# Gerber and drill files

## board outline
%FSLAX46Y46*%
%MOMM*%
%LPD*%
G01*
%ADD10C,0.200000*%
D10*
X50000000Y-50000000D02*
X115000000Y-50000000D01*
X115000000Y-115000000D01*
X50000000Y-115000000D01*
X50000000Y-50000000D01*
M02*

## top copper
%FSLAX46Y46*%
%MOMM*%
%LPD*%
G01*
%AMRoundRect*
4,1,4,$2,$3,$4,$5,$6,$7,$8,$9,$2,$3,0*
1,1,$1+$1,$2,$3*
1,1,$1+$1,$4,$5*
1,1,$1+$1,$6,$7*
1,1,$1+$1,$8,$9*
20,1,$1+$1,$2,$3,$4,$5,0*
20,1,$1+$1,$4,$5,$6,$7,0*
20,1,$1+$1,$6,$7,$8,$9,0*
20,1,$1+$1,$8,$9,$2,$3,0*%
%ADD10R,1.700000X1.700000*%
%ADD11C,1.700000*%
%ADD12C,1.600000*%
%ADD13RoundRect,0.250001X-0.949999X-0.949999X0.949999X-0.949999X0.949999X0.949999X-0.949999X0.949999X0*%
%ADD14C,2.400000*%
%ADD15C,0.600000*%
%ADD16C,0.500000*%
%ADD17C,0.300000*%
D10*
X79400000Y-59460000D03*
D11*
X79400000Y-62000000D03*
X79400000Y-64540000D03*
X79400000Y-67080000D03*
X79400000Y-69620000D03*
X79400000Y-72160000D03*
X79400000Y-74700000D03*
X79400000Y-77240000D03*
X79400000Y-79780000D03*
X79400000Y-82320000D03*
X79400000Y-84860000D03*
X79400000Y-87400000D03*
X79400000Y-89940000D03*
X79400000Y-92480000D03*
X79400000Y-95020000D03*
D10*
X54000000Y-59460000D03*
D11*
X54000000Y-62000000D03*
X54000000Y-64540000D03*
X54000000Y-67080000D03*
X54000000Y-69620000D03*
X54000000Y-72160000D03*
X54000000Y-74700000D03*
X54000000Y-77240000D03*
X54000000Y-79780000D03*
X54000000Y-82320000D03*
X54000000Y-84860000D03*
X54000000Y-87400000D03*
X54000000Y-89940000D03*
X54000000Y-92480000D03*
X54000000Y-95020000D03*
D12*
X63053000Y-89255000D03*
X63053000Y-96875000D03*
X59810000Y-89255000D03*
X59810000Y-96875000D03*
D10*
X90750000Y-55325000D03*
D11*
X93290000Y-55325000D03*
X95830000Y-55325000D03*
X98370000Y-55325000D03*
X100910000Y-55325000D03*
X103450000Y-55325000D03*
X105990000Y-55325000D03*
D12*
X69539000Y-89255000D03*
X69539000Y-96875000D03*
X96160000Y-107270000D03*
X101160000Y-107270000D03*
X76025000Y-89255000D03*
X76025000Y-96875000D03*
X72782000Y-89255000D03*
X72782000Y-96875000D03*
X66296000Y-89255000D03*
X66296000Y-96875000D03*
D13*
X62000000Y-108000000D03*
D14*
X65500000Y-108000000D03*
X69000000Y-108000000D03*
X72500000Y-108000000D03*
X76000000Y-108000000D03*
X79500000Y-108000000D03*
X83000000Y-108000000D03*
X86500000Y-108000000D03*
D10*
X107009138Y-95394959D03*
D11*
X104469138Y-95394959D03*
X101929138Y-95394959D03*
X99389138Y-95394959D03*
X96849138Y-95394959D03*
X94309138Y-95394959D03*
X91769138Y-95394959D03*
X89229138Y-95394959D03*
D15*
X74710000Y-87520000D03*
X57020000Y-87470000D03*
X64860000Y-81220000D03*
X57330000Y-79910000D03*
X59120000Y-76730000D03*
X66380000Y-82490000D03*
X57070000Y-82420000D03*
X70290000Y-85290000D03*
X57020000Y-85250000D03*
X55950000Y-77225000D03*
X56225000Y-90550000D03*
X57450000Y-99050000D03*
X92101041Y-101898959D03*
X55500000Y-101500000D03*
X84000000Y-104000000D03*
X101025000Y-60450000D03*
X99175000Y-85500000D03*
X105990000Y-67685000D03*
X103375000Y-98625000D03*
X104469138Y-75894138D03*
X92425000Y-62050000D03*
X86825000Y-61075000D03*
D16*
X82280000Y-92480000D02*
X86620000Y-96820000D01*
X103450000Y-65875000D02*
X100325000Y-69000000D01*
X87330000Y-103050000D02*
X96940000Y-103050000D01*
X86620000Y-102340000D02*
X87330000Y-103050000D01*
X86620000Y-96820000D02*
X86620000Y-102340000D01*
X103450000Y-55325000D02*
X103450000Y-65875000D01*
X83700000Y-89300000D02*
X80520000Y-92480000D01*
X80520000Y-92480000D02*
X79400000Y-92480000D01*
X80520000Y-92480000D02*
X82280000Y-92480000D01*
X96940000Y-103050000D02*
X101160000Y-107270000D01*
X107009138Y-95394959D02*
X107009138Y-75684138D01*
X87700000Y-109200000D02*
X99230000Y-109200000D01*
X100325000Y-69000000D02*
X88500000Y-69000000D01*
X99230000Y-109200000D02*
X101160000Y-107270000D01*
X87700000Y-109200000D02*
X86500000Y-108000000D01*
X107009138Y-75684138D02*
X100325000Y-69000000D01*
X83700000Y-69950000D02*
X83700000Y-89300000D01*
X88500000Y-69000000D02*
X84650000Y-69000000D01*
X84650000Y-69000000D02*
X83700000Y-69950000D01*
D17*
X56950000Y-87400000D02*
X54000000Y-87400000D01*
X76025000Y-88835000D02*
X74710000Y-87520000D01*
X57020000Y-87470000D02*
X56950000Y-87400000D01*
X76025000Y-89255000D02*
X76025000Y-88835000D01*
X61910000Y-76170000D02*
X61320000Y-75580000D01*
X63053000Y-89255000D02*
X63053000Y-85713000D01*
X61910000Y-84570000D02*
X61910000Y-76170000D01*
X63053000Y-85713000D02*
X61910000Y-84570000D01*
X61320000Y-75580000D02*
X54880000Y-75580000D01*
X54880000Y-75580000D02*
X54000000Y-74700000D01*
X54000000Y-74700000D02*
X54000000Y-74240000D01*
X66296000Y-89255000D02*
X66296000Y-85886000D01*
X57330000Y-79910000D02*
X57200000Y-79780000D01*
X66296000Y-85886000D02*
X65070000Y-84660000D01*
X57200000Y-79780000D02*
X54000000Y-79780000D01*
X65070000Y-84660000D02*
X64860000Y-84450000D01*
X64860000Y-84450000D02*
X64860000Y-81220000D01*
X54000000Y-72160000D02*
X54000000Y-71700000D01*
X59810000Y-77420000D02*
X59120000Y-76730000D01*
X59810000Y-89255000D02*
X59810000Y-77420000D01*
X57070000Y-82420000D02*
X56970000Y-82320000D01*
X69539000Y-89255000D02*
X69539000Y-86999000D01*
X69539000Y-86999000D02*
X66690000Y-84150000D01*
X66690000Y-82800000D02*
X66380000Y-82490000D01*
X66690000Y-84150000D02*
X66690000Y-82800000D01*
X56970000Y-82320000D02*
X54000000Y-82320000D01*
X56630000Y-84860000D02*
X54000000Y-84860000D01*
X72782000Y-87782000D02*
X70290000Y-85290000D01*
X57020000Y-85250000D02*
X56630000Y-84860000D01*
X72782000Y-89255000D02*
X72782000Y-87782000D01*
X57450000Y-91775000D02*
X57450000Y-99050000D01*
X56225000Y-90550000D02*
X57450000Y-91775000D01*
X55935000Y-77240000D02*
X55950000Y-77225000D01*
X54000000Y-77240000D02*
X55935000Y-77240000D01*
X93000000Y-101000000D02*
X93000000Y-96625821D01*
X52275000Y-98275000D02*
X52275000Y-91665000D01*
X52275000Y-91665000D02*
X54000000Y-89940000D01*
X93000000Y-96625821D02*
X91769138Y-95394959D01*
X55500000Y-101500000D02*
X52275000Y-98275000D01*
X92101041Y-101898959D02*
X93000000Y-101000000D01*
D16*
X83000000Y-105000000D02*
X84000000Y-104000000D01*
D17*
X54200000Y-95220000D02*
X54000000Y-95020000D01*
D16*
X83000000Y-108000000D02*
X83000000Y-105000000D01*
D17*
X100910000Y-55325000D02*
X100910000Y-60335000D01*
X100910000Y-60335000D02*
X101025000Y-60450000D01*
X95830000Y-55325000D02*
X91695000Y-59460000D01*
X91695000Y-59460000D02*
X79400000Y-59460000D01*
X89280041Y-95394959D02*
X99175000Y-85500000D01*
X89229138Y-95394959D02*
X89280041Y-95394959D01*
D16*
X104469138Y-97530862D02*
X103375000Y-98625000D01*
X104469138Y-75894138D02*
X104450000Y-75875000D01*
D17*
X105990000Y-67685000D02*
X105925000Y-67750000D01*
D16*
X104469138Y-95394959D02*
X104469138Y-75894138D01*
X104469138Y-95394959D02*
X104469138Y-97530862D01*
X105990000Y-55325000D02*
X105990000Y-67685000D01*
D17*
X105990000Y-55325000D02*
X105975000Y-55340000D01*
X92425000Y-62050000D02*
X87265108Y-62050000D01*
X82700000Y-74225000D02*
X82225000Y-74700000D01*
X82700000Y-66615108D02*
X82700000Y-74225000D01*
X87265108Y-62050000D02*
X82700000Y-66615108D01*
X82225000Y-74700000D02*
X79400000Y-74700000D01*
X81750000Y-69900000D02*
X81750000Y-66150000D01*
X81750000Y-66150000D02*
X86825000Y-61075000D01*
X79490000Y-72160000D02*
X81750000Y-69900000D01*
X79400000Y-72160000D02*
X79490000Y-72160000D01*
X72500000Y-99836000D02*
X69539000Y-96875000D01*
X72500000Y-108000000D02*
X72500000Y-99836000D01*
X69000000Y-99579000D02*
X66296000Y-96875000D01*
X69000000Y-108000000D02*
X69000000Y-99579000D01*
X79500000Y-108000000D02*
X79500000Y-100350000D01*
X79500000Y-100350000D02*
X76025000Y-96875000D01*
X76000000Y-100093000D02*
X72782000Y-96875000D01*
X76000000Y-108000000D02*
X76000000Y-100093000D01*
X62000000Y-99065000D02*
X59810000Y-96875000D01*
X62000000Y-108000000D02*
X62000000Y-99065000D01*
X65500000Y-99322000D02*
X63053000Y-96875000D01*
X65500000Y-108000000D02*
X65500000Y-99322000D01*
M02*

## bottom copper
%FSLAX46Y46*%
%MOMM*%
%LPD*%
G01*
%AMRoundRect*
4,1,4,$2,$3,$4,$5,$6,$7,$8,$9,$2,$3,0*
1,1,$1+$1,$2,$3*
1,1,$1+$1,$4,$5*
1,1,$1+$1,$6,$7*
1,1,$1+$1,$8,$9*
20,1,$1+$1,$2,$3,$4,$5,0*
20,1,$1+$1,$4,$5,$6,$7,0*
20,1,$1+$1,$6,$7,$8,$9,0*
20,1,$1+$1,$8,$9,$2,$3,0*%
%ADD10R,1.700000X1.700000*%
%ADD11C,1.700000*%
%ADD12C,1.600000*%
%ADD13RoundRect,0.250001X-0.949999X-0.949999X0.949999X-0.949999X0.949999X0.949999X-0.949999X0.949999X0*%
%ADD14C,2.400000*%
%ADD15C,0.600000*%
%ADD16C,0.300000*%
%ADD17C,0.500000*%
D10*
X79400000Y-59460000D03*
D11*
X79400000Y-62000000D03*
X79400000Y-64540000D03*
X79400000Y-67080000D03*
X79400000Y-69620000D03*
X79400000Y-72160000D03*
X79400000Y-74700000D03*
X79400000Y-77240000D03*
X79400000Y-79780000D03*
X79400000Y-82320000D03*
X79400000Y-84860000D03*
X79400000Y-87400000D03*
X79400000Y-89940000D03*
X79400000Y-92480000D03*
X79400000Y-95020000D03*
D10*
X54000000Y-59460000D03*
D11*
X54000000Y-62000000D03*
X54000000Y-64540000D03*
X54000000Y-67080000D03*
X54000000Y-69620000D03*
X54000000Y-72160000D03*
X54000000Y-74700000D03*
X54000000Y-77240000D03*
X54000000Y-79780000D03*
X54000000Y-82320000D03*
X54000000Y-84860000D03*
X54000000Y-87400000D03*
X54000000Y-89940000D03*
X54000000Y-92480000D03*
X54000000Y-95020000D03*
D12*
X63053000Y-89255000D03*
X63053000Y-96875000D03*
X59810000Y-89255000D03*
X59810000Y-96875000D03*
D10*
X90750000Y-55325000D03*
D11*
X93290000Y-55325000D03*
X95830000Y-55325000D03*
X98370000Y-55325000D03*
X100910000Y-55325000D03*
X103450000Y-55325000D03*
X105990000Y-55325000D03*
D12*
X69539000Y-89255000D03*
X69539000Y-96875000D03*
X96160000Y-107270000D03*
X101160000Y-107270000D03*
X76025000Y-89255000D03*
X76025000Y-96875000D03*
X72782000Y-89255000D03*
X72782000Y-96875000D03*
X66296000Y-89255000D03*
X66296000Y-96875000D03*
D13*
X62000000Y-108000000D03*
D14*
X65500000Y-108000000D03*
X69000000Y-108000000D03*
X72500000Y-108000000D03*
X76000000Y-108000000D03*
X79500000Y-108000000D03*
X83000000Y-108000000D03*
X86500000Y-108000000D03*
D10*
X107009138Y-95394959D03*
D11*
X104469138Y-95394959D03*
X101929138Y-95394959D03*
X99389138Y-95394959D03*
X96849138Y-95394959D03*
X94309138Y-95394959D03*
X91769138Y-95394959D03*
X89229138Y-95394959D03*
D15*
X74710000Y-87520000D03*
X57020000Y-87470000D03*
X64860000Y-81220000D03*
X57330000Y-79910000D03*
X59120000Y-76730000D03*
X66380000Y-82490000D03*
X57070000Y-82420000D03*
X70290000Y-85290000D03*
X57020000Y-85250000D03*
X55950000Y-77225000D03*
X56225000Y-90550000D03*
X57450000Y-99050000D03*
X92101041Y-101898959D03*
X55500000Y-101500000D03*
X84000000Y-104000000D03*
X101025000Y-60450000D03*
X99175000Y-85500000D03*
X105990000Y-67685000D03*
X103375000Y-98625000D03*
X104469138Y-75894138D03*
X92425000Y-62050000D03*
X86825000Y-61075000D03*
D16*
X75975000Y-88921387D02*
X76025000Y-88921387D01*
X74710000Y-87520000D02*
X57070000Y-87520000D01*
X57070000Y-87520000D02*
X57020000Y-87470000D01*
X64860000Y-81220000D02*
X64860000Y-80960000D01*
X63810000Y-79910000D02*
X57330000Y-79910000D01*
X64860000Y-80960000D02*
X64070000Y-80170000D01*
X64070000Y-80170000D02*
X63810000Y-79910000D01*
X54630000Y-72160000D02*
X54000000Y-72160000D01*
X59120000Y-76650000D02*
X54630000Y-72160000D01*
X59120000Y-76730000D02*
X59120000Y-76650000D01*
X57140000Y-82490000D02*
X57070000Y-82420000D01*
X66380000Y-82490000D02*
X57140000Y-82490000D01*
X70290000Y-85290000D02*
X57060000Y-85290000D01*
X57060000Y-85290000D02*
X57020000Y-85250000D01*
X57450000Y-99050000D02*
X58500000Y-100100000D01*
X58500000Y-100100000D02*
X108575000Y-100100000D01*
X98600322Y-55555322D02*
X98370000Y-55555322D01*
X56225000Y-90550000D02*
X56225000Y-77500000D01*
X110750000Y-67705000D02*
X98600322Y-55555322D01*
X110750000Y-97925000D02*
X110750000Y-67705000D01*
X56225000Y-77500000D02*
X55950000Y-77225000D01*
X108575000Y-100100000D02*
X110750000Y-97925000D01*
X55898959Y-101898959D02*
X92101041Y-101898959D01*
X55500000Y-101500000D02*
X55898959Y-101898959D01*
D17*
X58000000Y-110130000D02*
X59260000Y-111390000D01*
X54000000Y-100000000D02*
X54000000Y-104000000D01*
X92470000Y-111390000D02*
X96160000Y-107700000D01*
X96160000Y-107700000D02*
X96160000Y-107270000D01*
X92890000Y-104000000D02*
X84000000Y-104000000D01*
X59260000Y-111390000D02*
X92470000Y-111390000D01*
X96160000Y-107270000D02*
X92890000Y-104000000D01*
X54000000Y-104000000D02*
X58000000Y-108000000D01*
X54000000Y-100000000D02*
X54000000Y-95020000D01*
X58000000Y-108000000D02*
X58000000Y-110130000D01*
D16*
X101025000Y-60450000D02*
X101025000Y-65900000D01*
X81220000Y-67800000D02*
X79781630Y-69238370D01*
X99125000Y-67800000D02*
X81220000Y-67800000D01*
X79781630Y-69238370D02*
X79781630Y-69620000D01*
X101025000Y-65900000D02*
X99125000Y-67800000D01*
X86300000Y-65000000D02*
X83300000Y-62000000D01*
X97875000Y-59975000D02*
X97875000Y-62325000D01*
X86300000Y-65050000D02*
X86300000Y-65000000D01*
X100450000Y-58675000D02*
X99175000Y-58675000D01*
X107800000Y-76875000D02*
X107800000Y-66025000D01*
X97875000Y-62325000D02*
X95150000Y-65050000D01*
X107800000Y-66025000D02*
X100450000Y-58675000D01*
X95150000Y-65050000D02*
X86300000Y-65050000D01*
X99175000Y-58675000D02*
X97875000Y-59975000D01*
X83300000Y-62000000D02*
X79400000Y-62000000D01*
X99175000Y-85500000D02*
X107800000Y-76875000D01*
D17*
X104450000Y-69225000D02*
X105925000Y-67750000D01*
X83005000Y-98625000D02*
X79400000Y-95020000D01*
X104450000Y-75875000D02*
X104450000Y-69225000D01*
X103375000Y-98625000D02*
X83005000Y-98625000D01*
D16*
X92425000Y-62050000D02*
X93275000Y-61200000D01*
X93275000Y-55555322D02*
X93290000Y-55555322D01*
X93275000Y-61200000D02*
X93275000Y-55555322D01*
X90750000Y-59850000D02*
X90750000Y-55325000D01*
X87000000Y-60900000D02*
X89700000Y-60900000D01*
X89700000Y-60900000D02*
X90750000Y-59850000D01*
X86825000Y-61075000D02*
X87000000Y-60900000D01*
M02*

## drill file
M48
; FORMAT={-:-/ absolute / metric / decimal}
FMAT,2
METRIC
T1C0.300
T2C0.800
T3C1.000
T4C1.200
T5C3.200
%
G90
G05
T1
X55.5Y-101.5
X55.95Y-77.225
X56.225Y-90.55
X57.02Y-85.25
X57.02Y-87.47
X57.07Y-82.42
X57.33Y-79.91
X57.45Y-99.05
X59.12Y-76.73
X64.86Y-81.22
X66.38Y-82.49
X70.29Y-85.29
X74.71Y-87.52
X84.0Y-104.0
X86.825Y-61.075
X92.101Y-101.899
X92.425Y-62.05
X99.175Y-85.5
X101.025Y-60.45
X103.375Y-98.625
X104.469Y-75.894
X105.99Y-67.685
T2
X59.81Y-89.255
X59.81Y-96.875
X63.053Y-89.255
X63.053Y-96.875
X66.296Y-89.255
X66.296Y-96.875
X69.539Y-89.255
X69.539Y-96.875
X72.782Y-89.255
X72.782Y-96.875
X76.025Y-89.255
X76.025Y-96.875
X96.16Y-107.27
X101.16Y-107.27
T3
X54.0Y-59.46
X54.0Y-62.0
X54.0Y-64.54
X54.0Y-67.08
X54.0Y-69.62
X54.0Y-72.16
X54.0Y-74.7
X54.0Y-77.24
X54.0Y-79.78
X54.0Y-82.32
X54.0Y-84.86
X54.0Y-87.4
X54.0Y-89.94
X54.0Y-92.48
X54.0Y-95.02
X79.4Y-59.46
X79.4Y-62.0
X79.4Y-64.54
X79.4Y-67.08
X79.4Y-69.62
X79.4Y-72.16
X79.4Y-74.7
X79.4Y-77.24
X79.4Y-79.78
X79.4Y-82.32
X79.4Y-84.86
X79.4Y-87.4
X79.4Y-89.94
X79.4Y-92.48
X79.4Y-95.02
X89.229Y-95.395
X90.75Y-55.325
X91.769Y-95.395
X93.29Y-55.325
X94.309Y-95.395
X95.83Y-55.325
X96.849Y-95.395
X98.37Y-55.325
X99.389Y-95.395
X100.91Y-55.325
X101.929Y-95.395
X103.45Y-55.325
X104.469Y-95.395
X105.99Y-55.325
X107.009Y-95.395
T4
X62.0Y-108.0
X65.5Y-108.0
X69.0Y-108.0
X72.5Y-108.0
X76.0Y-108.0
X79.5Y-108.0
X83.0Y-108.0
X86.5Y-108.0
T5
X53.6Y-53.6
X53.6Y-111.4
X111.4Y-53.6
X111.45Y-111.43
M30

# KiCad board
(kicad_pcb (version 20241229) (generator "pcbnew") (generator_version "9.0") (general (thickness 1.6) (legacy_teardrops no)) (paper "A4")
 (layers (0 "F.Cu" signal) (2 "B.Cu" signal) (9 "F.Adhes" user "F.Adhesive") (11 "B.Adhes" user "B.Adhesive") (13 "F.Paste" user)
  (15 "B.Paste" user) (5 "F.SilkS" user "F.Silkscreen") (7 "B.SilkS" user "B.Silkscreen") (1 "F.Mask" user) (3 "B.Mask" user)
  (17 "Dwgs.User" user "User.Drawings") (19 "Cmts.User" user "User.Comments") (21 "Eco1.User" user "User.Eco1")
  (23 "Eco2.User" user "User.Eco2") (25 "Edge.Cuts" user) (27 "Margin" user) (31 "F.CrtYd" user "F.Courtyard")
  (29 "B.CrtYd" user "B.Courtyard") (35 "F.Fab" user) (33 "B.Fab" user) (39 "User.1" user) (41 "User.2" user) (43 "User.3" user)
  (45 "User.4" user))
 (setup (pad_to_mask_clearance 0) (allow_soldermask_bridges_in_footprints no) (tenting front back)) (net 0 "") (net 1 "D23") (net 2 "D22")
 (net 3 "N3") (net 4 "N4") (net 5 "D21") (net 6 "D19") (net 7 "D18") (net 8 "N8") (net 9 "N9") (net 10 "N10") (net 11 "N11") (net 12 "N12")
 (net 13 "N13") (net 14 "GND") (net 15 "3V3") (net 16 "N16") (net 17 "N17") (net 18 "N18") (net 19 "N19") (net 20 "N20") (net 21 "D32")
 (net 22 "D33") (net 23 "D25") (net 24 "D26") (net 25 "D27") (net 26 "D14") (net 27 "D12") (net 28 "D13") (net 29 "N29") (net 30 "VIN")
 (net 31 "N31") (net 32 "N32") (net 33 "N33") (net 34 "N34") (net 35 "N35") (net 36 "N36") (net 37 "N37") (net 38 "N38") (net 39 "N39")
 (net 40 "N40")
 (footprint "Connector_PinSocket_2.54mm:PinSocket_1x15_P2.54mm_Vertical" (layer "F.Cu") (at 79.4 59.46)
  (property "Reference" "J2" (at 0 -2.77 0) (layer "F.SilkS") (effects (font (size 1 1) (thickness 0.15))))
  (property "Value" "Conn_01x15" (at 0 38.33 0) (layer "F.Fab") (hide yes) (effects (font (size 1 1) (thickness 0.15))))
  (pad "1" thru_hole rect (at 0 0) (size 1.7 1.7) (drill 1) (layers "*.Cu" "*.Mask") (remove_unused_layers no) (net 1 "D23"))
  (pad "2" thru_hole circle (at 0 2.54) (size 1.7 1.7) (drill 1) (layers "*.Cu" "*.Mask") (remove_unused_layers no) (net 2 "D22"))
  (pad "3" thru_hole circle (at 0 5.08) (size 1.7 1.7) (drill 1) (layers "*.Cu" "*.Mask") (remove_unused_layers no) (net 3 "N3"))
  (pad "4" thru_hole circle (at 0 7.62) (size 1.7 1.7) (drill 1) (layers "*.Cu" "*.Mask") (remove_unused_layers no) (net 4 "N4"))
  (pad "5" thru_hole circle (at 0 10.16) (size 1.7 1.7) (drill 1) (layers "*.Cu" "*.Mask") (remove_unused_layers no) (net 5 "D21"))
  (pad "6" thru_hole circle (at 0 12.7) (size 1.7 1.7) (drill 1) (layers "*.Cu" "*.Mask") (remove_unused_layers no) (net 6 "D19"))
  (pad "7" thru_hole circle (at 0 15.24) (size 1.7 1.7) (drill 1) (layers "*.Cu" "*.Mask") (remove_unused_layers no) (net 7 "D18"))
  (pad "8" thru_hole circle (at 0 17.78) (size 1.7 1.7) (drill 1) (layers "*.Cu" "*.Mask") (remove_unused_layers no) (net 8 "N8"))
  (pad "9" thru_hole circle (at 0 20.32) (size 1.7 1.7) (drill 1) (layers "*.Cu" "*.Mask") (remove_unused_layers no) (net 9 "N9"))
  (pad "10" thru_hole circle (at 0 22.86) (size 1.7 1.7) (drill 1) (layers "*.Cu" "*.Mask") (remove_unused_layers no) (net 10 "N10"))
  (pad "11" thru_hole circle (at 0 25.4) (size 1.7 1.7) (drill 1) (layers "*.Cu" "*.Mask") (remove_unused_layers no) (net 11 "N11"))
  (pad "12" thru_hole circle (at 0 27.94) (size 1.7 1.7) (drill 1) (layers "*.Cu" "*.Mask") (remove_unused_layers no) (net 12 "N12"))
  (pad "13" thru_hole circle (at 0 30.48) (size 1.7 1.7) (drill 1) (layers "*.Cu" "*.Mask") (remove_unused_layers no) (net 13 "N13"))
  (pad "14" thru_hole circle (at 0 33.02) (size 1.7 1.7) (drill 1) (layers "*.Cu" "*.Mask") (remove_unused_layers no) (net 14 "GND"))
  (pad "15" thru_hole circle (at 0 35.56) (size 1.7 1.7) (drill 1) (layers "*.Cu" "*.Mask") (remove_unused_layers no) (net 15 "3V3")))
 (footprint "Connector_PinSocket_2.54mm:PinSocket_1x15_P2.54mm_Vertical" (layer "F.Cu") (at 54 59.46)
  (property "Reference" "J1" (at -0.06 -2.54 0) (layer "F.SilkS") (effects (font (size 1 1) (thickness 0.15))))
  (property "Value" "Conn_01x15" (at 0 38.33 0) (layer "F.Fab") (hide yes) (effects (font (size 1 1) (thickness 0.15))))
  (pad "1" thru_hole rect (at 0 0) (size 1.7 1.7) (drill 1) (layers "*.Cu" "*.Mask") (remove_unused_layers no) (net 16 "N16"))
  (pad "2" thru_hole circle (at 0 2.54) (size 1.7 1.7) (drill 1) (layers "*.Cu" "*.Mask") (remove_unused_layers no) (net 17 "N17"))
  (pad "3" thru_hole circle (at 0 5.08) (size 1.7 1.7) (drill 1) (layers "*.Cu" "*.Mask") (remove_unused_layers no) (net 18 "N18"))
  (pad "4" thru_hole circle (at 0 7.62) (size 1.7 1.7) (drill 1) (layers "*.Cu" "*.Mask") (remove_unused_layers no) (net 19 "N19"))
  (pad "5" thru_hole circle (at 0 10.16) (size 1.7 1.7) (drill 1) (layers "*.Cu" "*.Mask") (remove_unused_layers no) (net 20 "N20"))
  (pad "6" thru_hole circle (at 0 12.7) (size 1.7 1.7) (drill 1) (layers "*.Cu" "*.Mask") (remove_unused_layers no) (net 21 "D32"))
  (pad "7" thru_hole circle (at 0 15.24) (size 1.7 1.7) (drill 1) (layers "*.Cu" "*.Mask") (remove_unused_layers no) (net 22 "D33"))
  (pad "8" thru_hole circle (at 0 17.78) (size 1.7 1.7) (drill 1) (layers "*.Cu" "*.Mask") (remove_unused_layers no) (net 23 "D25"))
  (pad "9" thru_hole circle (at 0 20.32) (size 1.7 1.7) (drill 1) (layers "*.Cu" "*.Mask") (remove_unused_layers no) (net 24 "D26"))
  (pad "10" thru_hole circle (at 0 22.86) (size 1.7 1.7) (drill 1) (layers "*.Cu" "*.Mask") (remove_unused_layers no) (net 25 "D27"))
  (pad "11" thru_hole circle (at 0 25.4) (size 1.7 1.7) (drill 1) (layers "*.Cu" "*.Mask") (remove_unused_layers no) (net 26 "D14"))
  (pad "12" thru_hole circle (at 0 27.94) (size 1.7 1.7) (drill 1) (layers "*.Cu" "*.Mask") (remove_unused_layers no) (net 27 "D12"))
  (pad "13" thru_hole circle (at 0 30.48) (size 1.7 1.7) (drill 1) (layers "*.Cu" "*.Mask") (remove_unused_layers no) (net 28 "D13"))
  (pad "14" thru_hole circle (at 0 33.02) (size 1.7 1.7) (drill 1) (layers "*.Cu" "*.Mask") (remove_unused_layers no) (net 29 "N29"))
  (pad "15" thru_hole circle (at 0 35.56) (size 1.7 1.7) (drill 1) (layers "*.Cu" "*.Mask") (remove_unused_layers no) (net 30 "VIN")))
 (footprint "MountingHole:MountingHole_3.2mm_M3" (layer "F.Cu") (at 53.6 53.6)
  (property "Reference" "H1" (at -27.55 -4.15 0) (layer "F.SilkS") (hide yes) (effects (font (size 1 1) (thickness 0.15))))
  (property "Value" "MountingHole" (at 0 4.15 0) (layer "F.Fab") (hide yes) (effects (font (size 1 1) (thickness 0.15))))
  (pad "" np_thru_hole circle (at 0 0) (size 3.2 3.2) (drill 3.2) (layers "*.Cu" "*.Mask")))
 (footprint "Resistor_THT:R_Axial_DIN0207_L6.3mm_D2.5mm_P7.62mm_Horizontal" (layer "F.Cu") (at 63.053 89.255 -90)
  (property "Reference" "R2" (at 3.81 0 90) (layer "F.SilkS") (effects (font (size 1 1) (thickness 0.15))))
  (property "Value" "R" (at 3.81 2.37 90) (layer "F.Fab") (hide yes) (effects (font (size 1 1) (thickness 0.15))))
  (pad "1" thru_hole circle (at 0 0 270) (size 1.6 1.6) (drill 0.8) (layers "*.Cu" "*.Mask") (remove_unused_layers no) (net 22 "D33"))
  (pad "2" thru_hole circle (at 7.62 0 270) (size 1.6 1.6) (drill 0.8) (layers "*.Cu" "*.Mask") (remove_unused_layers no) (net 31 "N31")))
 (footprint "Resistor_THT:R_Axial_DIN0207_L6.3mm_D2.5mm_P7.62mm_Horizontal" (layer "F.Cu") (at 59.81 89.255 -90)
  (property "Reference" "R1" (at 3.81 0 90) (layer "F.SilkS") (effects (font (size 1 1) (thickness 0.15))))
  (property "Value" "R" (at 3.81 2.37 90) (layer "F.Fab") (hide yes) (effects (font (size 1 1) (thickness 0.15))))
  (pad "1" thru_hole circle (at 0 0 270) (size 1.6 1.6) (drill 0.8) (layers "*.Cu" "*.Mask") (remove_unused_layers no) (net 21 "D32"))
  (pad "2" thru_hole circle (at 7.62 0 270) (size 1.6 1.6) (drill 0.8) (layers "*.Cu" "*.Mask") (remove_unused_layers no) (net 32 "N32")))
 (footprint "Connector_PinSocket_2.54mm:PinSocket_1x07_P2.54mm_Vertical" (layer "F.Cu") (at 90.75 55.325 90)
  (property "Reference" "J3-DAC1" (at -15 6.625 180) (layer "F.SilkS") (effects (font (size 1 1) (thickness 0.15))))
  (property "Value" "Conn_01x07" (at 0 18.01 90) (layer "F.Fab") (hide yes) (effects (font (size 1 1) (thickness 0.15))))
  (pad "1" thru_hole rect (at 0 0 90) (size 1.7 1.7) (drill 1) (layers "*.Cu" "*.Mask") (remove_unused_layers no) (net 6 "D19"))
  (pad "2" thru_hole circle (at 0 2.54 90) (size 1.7 1.7) (drill 1) (layers "*.Cu" "*.Mask") (remove_unused_layers no) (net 7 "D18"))
  (pad "3" thru_hole circle (at 0 5.08 90) (size 1.7 1.7) (drill 1) (layers "*.Cu" "*.Mask") (remove_unused_layers no) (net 1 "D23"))
  (pad "4" thru_hole circle (at 0 7.62 90) (size 1.7 1.7) (drill 1) (layers "*.Cu" "*.Mask") (remove_unused_layers no) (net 23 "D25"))
  (pad "5" thru_hole circle (at 0 10.16 90) (size 1.7 1.7) (drill 1) (layers "*.Cu" "*.Mask") (remove_unused_layers no) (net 5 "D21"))
  (pad "6" thru_hole circle (at 0 12.7 90) (size 1.7 1.7) (drill 1) (layers "*.Cu" "*.Mask") (remove_unused_layers no) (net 14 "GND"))
  (pad "7" thru_hole circle (at 0 15.24 90) (size 1.7 1.7) (drill 1) (layers "*.Cu" "*.Mask") (remove_unused_layers no) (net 15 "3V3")))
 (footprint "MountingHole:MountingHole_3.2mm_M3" (layer "F.Cu") (at 53.6 111.4)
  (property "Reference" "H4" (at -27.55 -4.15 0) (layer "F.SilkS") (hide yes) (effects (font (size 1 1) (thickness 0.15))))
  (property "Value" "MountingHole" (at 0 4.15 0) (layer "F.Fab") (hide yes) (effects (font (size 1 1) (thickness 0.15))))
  (pad "" np_thru_hole circle (at 0 0) (size 3.2 3.2) (drill 3.2) (layers "*.Cu" "*.Mask")))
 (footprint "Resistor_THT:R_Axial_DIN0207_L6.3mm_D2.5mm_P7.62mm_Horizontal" (layer "F.Cu") (at 69.539 89.255 -90)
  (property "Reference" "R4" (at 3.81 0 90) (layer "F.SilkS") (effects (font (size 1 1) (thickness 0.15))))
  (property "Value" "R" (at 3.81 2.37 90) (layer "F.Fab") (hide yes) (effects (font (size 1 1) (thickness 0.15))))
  (pad "1" thru_hole circle (at 0 0 270) (size 1.6 1.6) (drill 0.8) (layers "*.Cu" "*.Mask") (remove_unused_layers no) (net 25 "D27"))
  (pad "2" thru_hole circle (at 7.62 0 270) (size 1.6 1.6) (drill 0.8) (layers "*.Cu" "*.Mask") (remove_unused_layers no) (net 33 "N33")))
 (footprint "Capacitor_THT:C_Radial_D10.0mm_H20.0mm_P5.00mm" (layer "F.Cu") (at 96.16 107.27)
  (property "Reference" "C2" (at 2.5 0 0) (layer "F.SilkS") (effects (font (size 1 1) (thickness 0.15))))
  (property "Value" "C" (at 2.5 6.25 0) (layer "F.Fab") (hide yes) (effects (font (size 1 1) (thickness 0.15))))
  (pad "1" thru_hole circle (at 0 0) (size 1.6 1.6) (drill 0.8) (layers "*.Cu" "*.Mask") (remove_unused_layers no) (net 30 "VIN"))
  (pad "2" thru_hole circle (at 5 0) (size 1.6 1.6) (drill 0.8) (layers "*.Cu" "*.Mask") (remove_unused_layers no) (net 14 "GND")))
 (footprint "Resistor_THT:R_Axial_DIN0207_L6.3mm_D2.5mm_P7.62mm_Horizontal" (layer "F.Cu") (at 76.025 89.255 -90)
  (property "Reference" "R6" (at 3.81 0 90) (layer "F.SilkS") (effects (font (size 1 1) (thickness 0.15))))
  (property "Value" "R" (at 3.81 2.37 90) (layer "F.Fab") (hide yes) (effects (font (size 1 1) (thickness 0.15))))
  (pad "1" thru_hole circle (at 0 0 270) (size 1.6 1.6) (drill 0.8) (layers "*.Cu" "*.Mask") (remove_unused_layers no) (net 27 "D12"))
  (pad "2" thru_hole circle (at 7.62 0 270) (size 1.6 1.6) (drill 0.8) (layers "*.Cu" "*.Mask") (remove_unused_layers no) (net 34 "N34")))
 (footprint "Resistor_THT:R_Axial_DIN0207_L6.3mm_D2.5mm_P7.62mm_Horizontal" (layer "F.Cu") (at 72.782 89.255 -90)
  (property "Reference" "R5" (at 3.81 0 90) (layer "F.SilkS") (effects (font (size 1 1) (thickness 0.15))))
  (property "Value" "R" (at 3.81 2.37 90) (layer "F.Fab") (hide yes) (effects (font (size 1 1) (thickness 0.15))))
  (pad "1" thru_hole circle (at 0 0 270) (size 1.6 1.6) (drill 0.8) (layers "*.Cu" "*.Mask") (remove_unused_layers no) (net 26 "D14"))
  (pad "2" thru_hole circle (at 7.62 0 270) (size 1.6 1.6) (drill 0.8) (layers "*.Cu" "*.Mask") (remove_unused_layers no) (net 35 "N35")))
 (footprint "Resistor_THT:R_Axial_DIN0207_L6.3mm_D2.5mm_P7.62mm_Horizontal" (layer "F.Cu") (at 66.296 89.255 -90)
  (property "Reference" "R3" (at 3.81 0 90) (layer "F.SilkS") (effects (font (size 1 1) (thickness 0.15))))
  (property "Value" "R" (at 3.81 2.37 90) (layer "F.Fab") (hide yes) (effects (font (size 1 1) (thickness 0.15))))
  (pad "1" thru_hole circle (at 0 0 270) (size 1.6 1.6) (drill 0.8) (layers "*.Cu" "*.Mask") (remove_unused_layers no) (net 24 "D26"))
  (pad "2" thru_hole circle (at 7.62 0 270) (size 1.6 1.6) (drill 0.8) (layers "*.Cu" "*.Mask") (remove_unused_layers no) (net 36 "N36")))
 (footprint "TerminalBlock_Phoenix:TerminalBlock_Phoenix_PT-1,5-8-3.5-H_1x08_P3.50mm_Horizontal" (layer "F.Cu") (at 62 108)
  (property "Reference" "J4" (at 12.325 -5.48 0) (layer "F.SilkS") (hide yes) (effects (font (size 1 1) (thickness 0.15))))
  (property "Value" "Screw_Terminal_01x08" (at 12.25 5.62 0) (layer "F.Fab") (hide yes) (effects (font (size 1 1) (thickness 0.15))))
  (pad "1" thru_hole roundrect (at 0 0) (size 2.4 2.4) (drill 1.2) (layers "*.Cu" "*.Mask") (remove_unused_layers no)
   (roundrect_rratio 0.104167) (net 32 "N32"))
  (pad "2" thru_hole circle (at 3.5 0) (size 2.4 2.4) (drill 1.2) (layers "*.Cu" "*.Mask") (remove_unused_layers no) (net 31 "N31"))
  (pad "3" thru_hole circle (at 7 0) (size 2.4 2.4) (drill 1.2) (layers "*.Cu" "*.Mask") (remove_unused_layers no) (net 36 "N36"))
  (pad "4" thru_hole circle (at 10.5 0) (size 2.4 2.4) (drill 1.2) (layers "*.Cu" "*.Mask") (remove_unused_layers no) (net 33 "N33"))
  (pad "5" thru_hole circle (at 14 0) (size 2.4 2.4) (drill 1.2) (layers "*.Cu" "*.Mask") (remove_unused_layers no) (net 35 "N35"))
  (pad "6" thru_hole circle (at 17.5 0) (size 2.4 2.4) (drill 1.2) (layers "*.Cu" "*.Mask") (remove_unused_layers no) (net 34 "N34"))
  (pad "7" thru_hole circle (at 21 0) (size 2.4 2.4) (drill 1.2) (layers "*.Cu" "*.Mask") (remove_unused_layers no) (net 30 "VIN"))
  (pad "8" thru_hole circle (at 24.5 0) (size 2.4 2.4) (drill 1.2) (layers "*.Cu" "*.Mask") (remove_unused_layers no) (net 14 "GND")))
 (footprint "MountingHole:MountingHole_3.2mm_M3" (layer "F.Cu") (at 111.45 111.43)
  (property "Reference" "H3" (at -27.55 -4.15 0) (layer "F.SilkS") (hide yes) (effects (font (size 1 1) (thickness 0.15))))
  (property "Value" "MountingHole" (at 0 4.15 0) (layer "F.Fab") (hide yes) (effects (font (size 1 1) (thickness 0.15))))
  (pad "" np_thru_hole circle (at 0 0) (size 3.2 3.2) (drill 3.2) (layers "*.Cu" "*.Mask")))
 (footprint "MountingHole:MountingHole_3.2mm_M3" (layer "F.Cu") (at 111.4 53.6)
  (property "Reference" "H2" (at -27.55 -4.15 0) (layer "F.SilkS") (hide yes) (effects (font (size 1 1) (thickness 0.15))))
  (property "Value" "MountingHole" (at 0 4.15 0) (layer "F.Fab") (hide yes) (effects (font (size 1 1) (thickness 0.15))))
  (pad "" np_thru_hole circle (at 0 0) (size 3.2 3.2) (drill 3.2) (layers "*.Cu" "*.Mask")))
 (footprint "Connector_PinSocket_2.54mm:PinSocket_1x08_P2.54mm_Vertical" (layer "F.Cu") (at 107.009138 95.394959 -90)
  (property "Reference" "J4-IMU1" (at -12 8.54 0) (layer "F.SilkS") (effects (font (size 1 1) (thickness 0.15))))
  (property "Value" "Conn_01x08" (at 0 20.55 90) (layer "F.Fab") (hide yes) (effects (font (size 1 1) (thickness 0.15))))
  (pad "1" thru_hole rect (at 0 0 270) (size 1.7 1.7) (drill 1) (layers "*.Cu" "*.Mask") (remove_unused_layers no) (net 14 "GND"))
  (pad "2" thru_hole circle (at 0 2.54 270) (size 1.7 1.7) (drill 1) (layers "*.Cu" "*.Mask") (remove_unused_layers no) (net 15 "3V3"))
  (pad "3" thru_hole circle (at 0 5.08 270) (size 1.7 1.7) (drill 1) (layers "*.Cu" "*.Mask") (remove_unused_layers no) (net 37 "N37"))
  (pad "4" thru_hole circle (at 0 7.62 270) (size 1.7 1.7) (drill 1) (layers "*.Cu" "*.Mask") (remove_unused_layers no) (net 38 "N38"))
  (pad "5" thru_hole circle (at 0 10.16 270) (size 1.7 1.7) (drill 1) (layers "*.Cu" "*.Mask") (remove_unused_layers no) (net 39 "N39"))
  (pad "6" thru_hole circle (at 0 12.7 270) (size 1.7 1.7) (drill 1) (layers "*.Cu" "*.Mask") (remove_unused_layers no) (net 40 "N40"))
  (pad "7" thru_hole circle (at 0 15.24 270) (size 1.7 1.7) (drill 1) (layers "*.Cu" "*.Mask") (remove_unused_layers no) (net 28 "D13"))
  (pad "8" thru_hole circle (at 0 17.78 270) (size 1.7 1.7) (drill 1) (layers "*.Cu" "*.Mask") (remove_unused_layers no) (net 2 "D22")))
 (gr_rect (start 50 50) (end 115 115) (stroke (width 0.2) (type solid)) (fill no) (layer "Edge.Cuts"))
 (segment (start 82.28 92.48) (end 86.62 96.82) (width 0.5) (layer "F.Cu") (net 14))
 (segment (start 103.45 65.875) (end 100.325 69) (width 0.5) (layer "F.Cu") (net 14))
 (segment (start 87.33 103.05) (end 96.94 103.05) (width 0.5) (layer "F.Cu") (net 14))
 (segment (start 86.62 102.34) (end 87.33 103.05) (width 0.5) (layer "F.Cu") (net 14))
 (segment (start 86.62 96.82) (end 86.62 102.34) (width 0.5) (layer "F.Cu") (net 14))
 (segment (start 103.45 55.325) (end 103.45 65.875) (width 0.5) (layer "F.Cu") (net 14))
 (segment (start 83.7 89.3) (end 80.52 92.48) (width 0.5) (layer "F.Cu") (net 14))
 (segment (start 80.52 92.48) (end 79.4 92.48) (width 0.5) (layer "F.Cu") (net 14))
 (segment (start 80.52 92.48) (end 82.28 92.48) (width 0.5) (layer "F.Cu") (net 14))
 (segment (start 96.94 103.05) (end 101.16 107.27) (width 0.5) (layer "F.Cu") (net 14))
 (segment (start 107.009138 95.394959) (end 107.009138 75.684138) (width 0.5) (layer "F.Cu") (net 14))
 (segment (start 87.7 109.2) (end 99.23 109.2) (width 0.5) (layer "F.Cu") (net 14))
 (segment (start 100.325 69) (end 88.5 69) (width 0.5) (layer "F.Cu") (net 14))
 (segment (start 99.23 109.2) (end 101.16 107.27) (width 0.5) (layer "F.Cu") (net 14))
 (segment (start 87.7 109.2) (end 86.5 108) (width 0.5) (layer "F.Cu") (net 14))
 (segment (start 107.009138 75.684138) (end 100.325 69) (width 0.5) (layer "F.Cu") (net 14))
 (segment (start 83.7 69.95) (end 83.7 89.3) (width 0.5) (layer "F.Cu") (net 14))
 (segment (start 88.5 69) (end 84.65 69) (width 0.5) (layer "F.Cu") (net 14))
 (segment (start 84.65 69) (end 83.7 69.95) (width 0.5) (layer "F.Cu") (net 14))
 (segment (start 56.95 87.4) (end 54 87.4) (width 0.3) (layer "F.Cu") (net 27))
 (segment (start 76.025 88.835) (end 74.71 87.52) (width 0.3) (layer "F.Cu") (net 27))
 (segment (start 57.02 87.47) (end 56.95 87.4) (width 0.3) (layer "F.Cu") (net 27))
 (segment (start 76.025 89.255) (end 76.025 88.835) (width 0.3) (layer "F.Cu") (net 27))
 (via (at 74.71 87.52) (size 0.6) (drill 0.3) (layers "F.Cu" "B.Cu") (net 27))
 (via (at 57.02 87.47) (size 0.6) (drill 0.3) (layers "F.Cu" "B.Cu") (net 27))
 (segment (start 75.975 88.921387) (end 76.025 88.921387) (width 0.3) (layer "B.Cu") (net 27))
 (segment (start 74.71 87.52) (end 57.07 87.52) (width 0.3) (layer "B.Cu") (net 27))
 (segment (start 57.07 87.52) (end 57.02 87.47) (width 0.3) (layer "B.Cu") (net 27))
 (segment (start 61.91 76.17) (end 61.32 75.58) (width 0.3) (layer "F.Cu") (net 22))
 (segment (start 63.053 89.255) (end 63.053 85.713) (width 0.3) (layer "F.Cu") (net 22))
 (segment (start 61.91 84.57) (end 61.91 76.17) (width 0.3) (layer "F.Cu") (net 22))
 (segment (start 63.053 85.713) (end 61.91 84.57) (width 0.3) (layer "F.Cu") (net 22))
 (segment (start 61.32 75.58) (end 54.88 75.58) (width 0.3) (layer "F.Cu") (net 22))
 (segment (start 54.88 75.58) (end 54 74.7) (width 0.3) (layer "F.Cu") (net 22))
 (segment (start 54 74.7) (end 54 74.24) (width 0.3) (layer "F.Cu") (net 22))
 (segment (start 66.296 89.255) (end 66.296 85.886) (width 0.3) (layer "F.Cu") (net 24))
 (segment (start 57.33 79.91) (end 57.2 79.78) (width 0.3) (layer "F.Cu") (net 24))
 (segment (start 66.296 85.886) (end 65.07 84.66) (width 0.3) (layer "F.Cu") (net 24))
 (segment (start 57.2 79.78) (end 54 79.78) (width 0.3) (layer "F.Cu") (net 24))
 (segment (start 65.07 84.66) (end 64.86 84.45) (width 0.3) (layer "F.Cu") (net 24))
 (segment (start 64.86 84.45) (end 64.86 81.22) (width 0.3) (layer "F.Cu") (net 24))
 (via (at 64.86 81.22) (size 0.6) (drill 0.3) (layers "F.Cu" "B.Cu") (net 24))
 (via (at 57.33 79.91) (size 0.6) (drill 0.3) (layers "F.Cu" "B.Cu") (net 24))
 (segment (start 64.86 81.22) (end 64.86 80.96) (width 0.3) (layer "B.Cu") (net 24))
 (segment (start 63.81 79.91) (end 57.33 79.91) (width 0.3) (layer "B.Cu") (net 24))
 (segment (start 64.86 80.96) (end 64.07 80.17) (width 0.3) (layer "B.Cu") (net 24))
 (segment (start 64.07 80.17) (end 63.81 79.91) (width 0.3) (layer "B.Cu") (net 24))
 (segment (start 54 72.16) (end 54 71.7) (width 0.3) (layer "F.Cu") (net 21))
 (segment (start 59.81 77.42) (end 59.12 76.73) (width 0.3) (layer "F.Cu") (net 21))
 (segment (start 59.81 89.255) (end 59.81 77.42) (width 0.3) (layer "F.Cu") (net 21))
 (via (at 59.12 76.73) (size 0.6) (drill 0.3) (layers "F.Cu" "B.Cu") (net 21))
 (segment (start 54.63 72.16) (end 54 72.16) (width 0.3) (layer "B.Cu") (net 21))
 (segment (start 59.12 76.65) (end 54.63 72.16) (width 0.3) (layer "B.Cu") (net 21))
 (segment (start 59.12 76.73) (end 59.12 76.65) (width 0.3) (layer "B.Cu") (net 21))
 (segment (start 57.07 82.42) (end 56.97 82.32) (width 0.3) (layer "F.Cu") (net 25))
 (segment (start 69.539 89.255) (end 69.539 86.999) (width 0.3) (layer "F.Cu") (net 25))
 (segment (start 69.539 86.999) (end 66.69 84.15) (width 0.3) (layer "F.Cu") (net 25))
 (segment (start 66.69 82.8) (end 66.38 82.49) (width 0.3) (layer "F.Cu") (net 25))
 (segment (start 66.69 84.15) (end 66.69 82.8) (width 0.3) (layer "F.Cu") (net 25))
 (segment (start 56.97 82.32) (end 54 82.32) (width 0.3) (layer "F.Cu") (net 25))
 (via (at 66.38 82.49) (size 0.6) (drill 0.3) (layers "F.Cu" "B.Cu") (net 25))
 (via (at 57.07 82.42) (size 0.6) (drill 0.3) (layers "F.Cu" "B.Cu") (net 25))
 (segment (start 57.14 82.49) (end 57.07 82.42) (width 0.3) (layer "B.Cu") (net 25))
 (segment (start 66.38 82.49) (end 57.14 82.49) (width 0.3) (layer "B.Cu") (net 25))
 (segment (start 56.63 84.86) (end 54 84.86) (width 0.3) (layer "F.Cu") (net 26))
 (segment (start 72.782 87.782) (end 70.29 85.29) (width 0.3) (layer "F.Cu") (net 26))
 (segment (start 57.02 85.25) (end 56.63 84.86) (width 0.3) (layer "F.Cu") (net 26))
 (segment (start 72.782 89.255) (end 72.782 87.782) (width 0.3) (layer "F.Cu") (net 26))
 (via (at 70.29 85.29) (size 0.6) (drill 0.3) (layers "F.Cu" "B.Cu") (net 26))
 (via (at 57.02 85.25) (size 0.6) (drill 0.3) (layers "F.Cu" "B.Cu") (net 26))
 (segment (start 70.29 85.29) (end 57.06 85.29) (width 0.3) (layer "B.Cu") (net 26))
 (segment (start 57.06 85.29) (end 57.02 85.25) (width 0.3) (layer "B.Cu") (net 26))
 (segment (start 57.45 91.775) (end 57.45 99.05) (width 0.3) (layer "F.Cu") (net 23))
 (segment (start 56.225 90.55) (end 57.45 91.775) (width 0.3) (layer "F.Cu") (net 23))
 (segment (start 55.935 77.24) (end 55.95 77.225) (width 0.3) (layer "F.Cu") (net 23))
 (segment (start 54 77.24) (end 55.935 77.24) (width 0.3) (layer "F.Cu") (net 23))
 (via (at 55.95 77.225) (size 0.6) (drill 0.3) (layers "F.Cu" "B.Cu") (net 23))
 (via (at 56.225 90.55) (size 0.6) (drill 0.3) (layers "F.Cu" "B.Cu") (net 23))
 (via (at 57.45 99.05) (size 0.6) (drill 0.3) (layers "F.Cu" "B.Cu") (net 23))
 (segment (start 57.45 99.05) (end 58.5 100.1) (width 0.3) (layer "B.Cu") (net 23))
 (segment (start 58.5 100.1) (end 108.575 100.1) (width 0.3) (layer "B.Cu") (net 23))
 (segment (start 98.600322 55.555322) (end 98.37 55.555322) (width 0.3) (layer "B.Cu") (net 23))
 (segment (start 56.225 90.55) (end 56.225 77.5) (width 0.3) (layer "B.Cu") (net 23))
 (segment (start 110.75 67.705) (end 98.600322 55.555322) (width 0.3) (layer "B.Cu") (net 23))
 (segment (start 110.75 97.925) (end 110.75 67.705) (width 0.3) (layer "B.Cu") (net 23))
 (segment (start 56.225 77.5) (end 55.95 77.225) (width 0.3) (layer "B.Cu") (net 23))
 (segment (start 108.575 100.1) (end 110.75 97.925) (width 0.3) (layer "B.Cu") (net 23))
 (segment (start 93 101) (end 93 96.625821) (width 0.3) (layer "F.Cu") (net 28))
 (segment (start 52.275 98.275) (end 52.275 91.665) (width 0.3) (layer "F.Cu") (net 28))
 (segment (start 52.275 91.665) (end 54 89.94) (width 0.3) (layer "F.Cu") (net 28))
 (segment (start 93 96.625821) (end 91.769138 95.394959) (width 0.3) (layer "F.Cu") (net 28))
 (segment (start 55.5 101.5) (end 52.275 98.275) (width 0.3) (layer "F.Cu") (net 28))
 (segment (start 92.101041 101.898959) (end 93 101) (width 0.3) (layer "F.Cu") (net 28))
 (via (at 92.101041 101.898959) (size 0.6) (drill 0.3) (layers "F.Cu" "B.Cu") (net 28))
 (via (at 55.5 101.5) (size 0.6) (drill 0.3) (layers "F.Cu" "B.Cu") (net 28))
 (segment (start 55.898959 101.898959) (end 92.101041 101.898959) (width 0.3) (layer "B.Cu") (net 28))
 (segment (start 55.5 101.5) (end 55.898959 101.898959) (width 0.3) (layer "B.Cu") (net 28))
 (segment (start 83 105) (end 84 104) (width 0.5) (layer "F.Cu") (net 30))
 (segment (start 54.2 95.22) (end 54 95.02) (width 0.3) (layer "F.Cu") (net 30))
 (segment (start 83 108) (end 83 105) (width 0.5) (layer "F.Cu") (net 30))
 (via (at 84 104) (size 0.6) (drill 0.3) (layers "F.Cu" "B.Cu") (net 30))
 (segment (start 58 110.13) (end 59.26 111.39) (width 0.5) (layer "B.Cu") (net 30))
 (segment (start 54 100) (end 54 104) (width 0.5) (layer "B.Cu") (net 30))
 (segment (start 92.47 111.39) (end 96.16 107.7) (width 0.5) (layer "B.Cu") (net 30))
 (segment (start 96.16 107.7) (end 96.16 107.27) (width 0.5) (layer "B.Cu") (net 30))
 (segment (start 92.89 104) (end 84 104) (width 0.5) (layer "B.Cu") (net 30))
 (segment (start 59.26 111.39) (end 92.47 111.39) (width 0.5) (layer "B.Cu") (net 30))
 (segment (start 96.16 107.27) (end 92.89 104) (width 0.5) (layer "B.Cu") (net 30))
 (segment (start 54 104) (end 58 108) (width 0.5) (layer "B.Cu") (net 30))
 (segment (start 54 100) (end 54 95.02) (width 0.5) (layer "B.Cu") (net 30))
 (segment (start 58 108) (end 58 110.13) (width 0.5) (layer "B.Cu") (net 30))
 (segment (start 100.91 55.325) (end 100.91 60.335) (width 0.3) (layer "F.Cu") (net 5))
 (segment (start 100.91 60.335) (end 101.025 60.45) (width 0.3) (layer "F.Cu") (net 5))
 (via (at 101.025 60.45) (size 0.6) (drill 0.3) (layers "F.Cu" "B.Cu") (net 5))
 (segment (start 101.025 60.45) (end 101.025 65.9) (width 0.3) (layer "B.Cu") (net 5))
 (segment (start 81.22 67.8) (end 79.78163 69.23837) (width 0.3) (layer "B.Cu") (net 5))
 (segment (start 99.125 67.8) (end 81.22 67.8) (width 0.3) (layer "B.Cu") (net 5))
 (segment (start 79.78163 69.23837) (end 79.78163 69.62) (width 0.3) (layer "B.Cu") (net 5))
 (segment (start 101.025 65.9) (end 99.125 67.8) (width 0.3) (layer "B.Cu") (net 5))
 (segment (start 95.83 55.325) (end 91.695 59.46) (width 0.3) (layer "F.Cu") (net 1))
 (segment (start 91.695 59.46) (end 79.4 59.46) (width 0.3) (layer "F.Cu") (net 1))
 (segment (start 89.280041 95.394959) (end 99.175 85.5) (width 0.3) (layer "F.Cu") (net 2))
 (segment (start 89.229138 95.394959) (end 89.280041 95.394959) (width 0.3) (layer "F.Cu") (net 2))
 (via (at 99.175 85.5) (size 0.6) (drill 0.3) (layers "F.Cu" "B.Cu") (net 2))
 (segment (start 86.3 65) (end 83.3 62) (width 0.3) (layer "B.Cu") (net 2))
 (segment (start 97.875 59.975) (end 97.875 62.325) (width 0.3) (layer "B.Cu") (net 2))
 (segment (start 86.3 65.05) (end 86.3 65) (width 0.3) (layer "B.Cu") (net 2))
 (segment (start 100.45 58.675) (end 99.175 58.675) (width 0.3) (layer "B.Cu") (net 2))
 (segment (start 107.8 76.875) (end 107.8 66.025) (width 0.3) (layer "B.Cu") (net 2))
 (segment (start 97.875 62.325) (end 95.15 65.05) (width 0.3) (layer "B.Cu") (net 2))
 (segment (start 107.8 66.025) (end 100.45 58.675) (width 0.3) (layer "B.Cu") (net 2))
 (segment (start 95.15 65.05) (end 86.3 65.05) (width 0.3) (layer "B.Cu") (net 2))
 (segment (start 99.175 58.675) (end 97.875 59.975) (width 0.3) (layer "B.Cu") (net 2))
 (segment (start 83.3 62) (end 79.4 62) (width 0.3) (layer "B.Cu") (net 2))
 (segment (start 99.175 85.5) (end 107.8 76.875) (width 0.3) (layer "B.Cu") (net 2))
 (segment (start 104.469138 97.530862) (end 103.375 98.625) (width 0.5) (layer "F.Cu") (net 15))
 (segment (start 104.469138 75.894138) (end 104.45 75.875) (width 0.5) (layer "F.Cu") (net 15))
 (segment (start 105.99 67.685) (end 105.925 67.75) (width 0.3) (layer "F.Cu") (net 15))
 (segment (start 104.469138 95.394959) (end 104.469138 75.894138) (width 0.5) (layer "F.Cu") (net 15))
 (segment (start 104.469138 95.394959) (end 104.469138 97.530862) (width 0.5) (layer "F.Cu") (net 15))
 (segment (start 105.99 55.325) (end 105.99 67.685) (width 0.5) (layer "F.Cu") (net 15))
 (segment (start 105.99 55.325) (end 105.975 55.34) (width 0.3) (layer "F.Cu") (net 15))
 (via (at 105.99 67.685) (size 0.6) (drill 0.3) (layers "F.Cu" "B.Cu") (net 15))
 (via (at 103.375 98.625) (size 0.6) (drill 0.3) (layers "F.Cu" "B.Cu") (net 15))
 (via (at 104.469138 75.894138) (size 0.6) (drill 0.3) (layers "F.Cu" "B.Cu") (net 15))
 (segment (start 104.45 69.225) (end 105.925 67.75) (width 0.5) (layer "B.Cu") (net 15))
 (segment (start 83.005 98.625) (end 79.4 95.02) (width 0.5) (layer "B.Cu") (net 15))
 (segment (start 104.45 75.875) (end 104.45 69.225) (width 0.5) (layer "B.Cu") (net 15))
 (segment (start 103.375 98.625) (end 83.005 98.625) (width 0.5) (layer "B.Cu") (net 15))
 (segment (start 92.425 62.05) (end 87.265108 62.05) (width 0.3) (layer "F.Cu") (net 7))
 (segment (start 82.7 74.225) (end 82.225 74.7) (width 0.3) (layer "F.Cu") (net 7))
 (segment (start 82.7 66.615108) (end 82.7 74.225) (width 0.3) (layer "F.Cu") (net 7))
 (segment (start 87.265108 62.05) (end 82.7 66.615108) (width 0.3) (layer "F.Cu") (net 7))
 (segment (start 82.225 74.7) (end 79.4 74.7) (width 0.3) (layer "F.Cu") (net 7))
 (via (at 92.425 62.05) (size 0.6) (drill 0.3) (layers "F.Cu" "B.Cu") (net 7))
 (segment (start 92.425 62.05) (end 93.275 61.2) (width 0.3) (layer "B.Cu") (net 7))
 (segment (start 93.275 55.555322) (end 93.29 55.555322) (width 0.3) (layer "B.Cu") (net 7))
 (segment (start 93.275 61.2) (end 93.275 55.555322) (width 0.3) (layer "B.Cu") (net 7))
 (segment (start 81.75 69.9) (end 81.75 66.15) (width 0.3) (layer "F.Cu") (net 6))
 (segment (start 81.75 66.15) (end 86.825 61.075) (width 0.3) (layer "F.Cu") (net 6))
 (segment (start 79.49 72.16) (end 81.75 69.9) (width 0.3) (layer "F.Cu") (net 6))
 (segment (start 79.4 72.16) (end 79.49 72.16) (width 0.3) (layer "F.Cu") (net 6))
 (via (at 86.825 61.075) (size 0.6) (drill 0.3) (layers "F.Cu" "B.Cu") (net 6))
 (segment (start 90.75 59.85) (end 90.75 55.325) (width 0.3) (layer "B.Cu") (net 6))
 (segment (start 87 60.9) (end 89.7 60.9) (width 0.3) (layer "B.Cu") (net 6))
 (segment (start 89.7 60.9) (end 90.75 59.85) (width 0.3) (layer "B.Cu") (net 6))
 (segment (start 86.825 61.075) (end 87 60.9) (width 0.3) (layer "B.Cu") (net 6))
 (segment (start 72.5 99.836) (end 69.539 96.875) (width 0.3) (layer "F.Cu") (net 33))
 (segment (start 72.5 108) (end 72.5 99.836) (width 0.3) (layer "F.Cu") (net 33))
 (segment (start 69 99.579) (end 66.296 96.875) (width 0.3) (layer "F.Cu") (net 36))
 (segment (start 69 108) (end 69 99.579) (width 0.3) (layer "F.Cu") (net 36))
 (segment (start 79.5 108) (end 79.5 100.35) (width 0.3) (layer "F.Cu") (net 34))
 (segment (start 79.5 100.35) (end 76.025 96.875) (width 0.3) (layer "F.Cu") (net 34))
 (segment (start 76 100.093) (end 72.782 96.875) (width 0.3) (layer "F.Cu") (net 35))
 (segment (start 76 108) (end 76 100.093) (width 0.3) (layer "F.Cu") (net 35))
 (segment (start 62 99.065) (end 59.81 96.875) (width 0.3) (layer "F.Cu") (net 32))
 (segment (start 62 108) (end 62 99.065) (width 0.3) (layer "F.Cu") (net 32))
 (segment (start 65.5 99.322) (end 63.053 96.875) (width 0.3) (layer "F.Cu") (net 31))
 (segment (start 65.5 108) (end 65.5 99.322) (width 0.3) (layer "F.Cu") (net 31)))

